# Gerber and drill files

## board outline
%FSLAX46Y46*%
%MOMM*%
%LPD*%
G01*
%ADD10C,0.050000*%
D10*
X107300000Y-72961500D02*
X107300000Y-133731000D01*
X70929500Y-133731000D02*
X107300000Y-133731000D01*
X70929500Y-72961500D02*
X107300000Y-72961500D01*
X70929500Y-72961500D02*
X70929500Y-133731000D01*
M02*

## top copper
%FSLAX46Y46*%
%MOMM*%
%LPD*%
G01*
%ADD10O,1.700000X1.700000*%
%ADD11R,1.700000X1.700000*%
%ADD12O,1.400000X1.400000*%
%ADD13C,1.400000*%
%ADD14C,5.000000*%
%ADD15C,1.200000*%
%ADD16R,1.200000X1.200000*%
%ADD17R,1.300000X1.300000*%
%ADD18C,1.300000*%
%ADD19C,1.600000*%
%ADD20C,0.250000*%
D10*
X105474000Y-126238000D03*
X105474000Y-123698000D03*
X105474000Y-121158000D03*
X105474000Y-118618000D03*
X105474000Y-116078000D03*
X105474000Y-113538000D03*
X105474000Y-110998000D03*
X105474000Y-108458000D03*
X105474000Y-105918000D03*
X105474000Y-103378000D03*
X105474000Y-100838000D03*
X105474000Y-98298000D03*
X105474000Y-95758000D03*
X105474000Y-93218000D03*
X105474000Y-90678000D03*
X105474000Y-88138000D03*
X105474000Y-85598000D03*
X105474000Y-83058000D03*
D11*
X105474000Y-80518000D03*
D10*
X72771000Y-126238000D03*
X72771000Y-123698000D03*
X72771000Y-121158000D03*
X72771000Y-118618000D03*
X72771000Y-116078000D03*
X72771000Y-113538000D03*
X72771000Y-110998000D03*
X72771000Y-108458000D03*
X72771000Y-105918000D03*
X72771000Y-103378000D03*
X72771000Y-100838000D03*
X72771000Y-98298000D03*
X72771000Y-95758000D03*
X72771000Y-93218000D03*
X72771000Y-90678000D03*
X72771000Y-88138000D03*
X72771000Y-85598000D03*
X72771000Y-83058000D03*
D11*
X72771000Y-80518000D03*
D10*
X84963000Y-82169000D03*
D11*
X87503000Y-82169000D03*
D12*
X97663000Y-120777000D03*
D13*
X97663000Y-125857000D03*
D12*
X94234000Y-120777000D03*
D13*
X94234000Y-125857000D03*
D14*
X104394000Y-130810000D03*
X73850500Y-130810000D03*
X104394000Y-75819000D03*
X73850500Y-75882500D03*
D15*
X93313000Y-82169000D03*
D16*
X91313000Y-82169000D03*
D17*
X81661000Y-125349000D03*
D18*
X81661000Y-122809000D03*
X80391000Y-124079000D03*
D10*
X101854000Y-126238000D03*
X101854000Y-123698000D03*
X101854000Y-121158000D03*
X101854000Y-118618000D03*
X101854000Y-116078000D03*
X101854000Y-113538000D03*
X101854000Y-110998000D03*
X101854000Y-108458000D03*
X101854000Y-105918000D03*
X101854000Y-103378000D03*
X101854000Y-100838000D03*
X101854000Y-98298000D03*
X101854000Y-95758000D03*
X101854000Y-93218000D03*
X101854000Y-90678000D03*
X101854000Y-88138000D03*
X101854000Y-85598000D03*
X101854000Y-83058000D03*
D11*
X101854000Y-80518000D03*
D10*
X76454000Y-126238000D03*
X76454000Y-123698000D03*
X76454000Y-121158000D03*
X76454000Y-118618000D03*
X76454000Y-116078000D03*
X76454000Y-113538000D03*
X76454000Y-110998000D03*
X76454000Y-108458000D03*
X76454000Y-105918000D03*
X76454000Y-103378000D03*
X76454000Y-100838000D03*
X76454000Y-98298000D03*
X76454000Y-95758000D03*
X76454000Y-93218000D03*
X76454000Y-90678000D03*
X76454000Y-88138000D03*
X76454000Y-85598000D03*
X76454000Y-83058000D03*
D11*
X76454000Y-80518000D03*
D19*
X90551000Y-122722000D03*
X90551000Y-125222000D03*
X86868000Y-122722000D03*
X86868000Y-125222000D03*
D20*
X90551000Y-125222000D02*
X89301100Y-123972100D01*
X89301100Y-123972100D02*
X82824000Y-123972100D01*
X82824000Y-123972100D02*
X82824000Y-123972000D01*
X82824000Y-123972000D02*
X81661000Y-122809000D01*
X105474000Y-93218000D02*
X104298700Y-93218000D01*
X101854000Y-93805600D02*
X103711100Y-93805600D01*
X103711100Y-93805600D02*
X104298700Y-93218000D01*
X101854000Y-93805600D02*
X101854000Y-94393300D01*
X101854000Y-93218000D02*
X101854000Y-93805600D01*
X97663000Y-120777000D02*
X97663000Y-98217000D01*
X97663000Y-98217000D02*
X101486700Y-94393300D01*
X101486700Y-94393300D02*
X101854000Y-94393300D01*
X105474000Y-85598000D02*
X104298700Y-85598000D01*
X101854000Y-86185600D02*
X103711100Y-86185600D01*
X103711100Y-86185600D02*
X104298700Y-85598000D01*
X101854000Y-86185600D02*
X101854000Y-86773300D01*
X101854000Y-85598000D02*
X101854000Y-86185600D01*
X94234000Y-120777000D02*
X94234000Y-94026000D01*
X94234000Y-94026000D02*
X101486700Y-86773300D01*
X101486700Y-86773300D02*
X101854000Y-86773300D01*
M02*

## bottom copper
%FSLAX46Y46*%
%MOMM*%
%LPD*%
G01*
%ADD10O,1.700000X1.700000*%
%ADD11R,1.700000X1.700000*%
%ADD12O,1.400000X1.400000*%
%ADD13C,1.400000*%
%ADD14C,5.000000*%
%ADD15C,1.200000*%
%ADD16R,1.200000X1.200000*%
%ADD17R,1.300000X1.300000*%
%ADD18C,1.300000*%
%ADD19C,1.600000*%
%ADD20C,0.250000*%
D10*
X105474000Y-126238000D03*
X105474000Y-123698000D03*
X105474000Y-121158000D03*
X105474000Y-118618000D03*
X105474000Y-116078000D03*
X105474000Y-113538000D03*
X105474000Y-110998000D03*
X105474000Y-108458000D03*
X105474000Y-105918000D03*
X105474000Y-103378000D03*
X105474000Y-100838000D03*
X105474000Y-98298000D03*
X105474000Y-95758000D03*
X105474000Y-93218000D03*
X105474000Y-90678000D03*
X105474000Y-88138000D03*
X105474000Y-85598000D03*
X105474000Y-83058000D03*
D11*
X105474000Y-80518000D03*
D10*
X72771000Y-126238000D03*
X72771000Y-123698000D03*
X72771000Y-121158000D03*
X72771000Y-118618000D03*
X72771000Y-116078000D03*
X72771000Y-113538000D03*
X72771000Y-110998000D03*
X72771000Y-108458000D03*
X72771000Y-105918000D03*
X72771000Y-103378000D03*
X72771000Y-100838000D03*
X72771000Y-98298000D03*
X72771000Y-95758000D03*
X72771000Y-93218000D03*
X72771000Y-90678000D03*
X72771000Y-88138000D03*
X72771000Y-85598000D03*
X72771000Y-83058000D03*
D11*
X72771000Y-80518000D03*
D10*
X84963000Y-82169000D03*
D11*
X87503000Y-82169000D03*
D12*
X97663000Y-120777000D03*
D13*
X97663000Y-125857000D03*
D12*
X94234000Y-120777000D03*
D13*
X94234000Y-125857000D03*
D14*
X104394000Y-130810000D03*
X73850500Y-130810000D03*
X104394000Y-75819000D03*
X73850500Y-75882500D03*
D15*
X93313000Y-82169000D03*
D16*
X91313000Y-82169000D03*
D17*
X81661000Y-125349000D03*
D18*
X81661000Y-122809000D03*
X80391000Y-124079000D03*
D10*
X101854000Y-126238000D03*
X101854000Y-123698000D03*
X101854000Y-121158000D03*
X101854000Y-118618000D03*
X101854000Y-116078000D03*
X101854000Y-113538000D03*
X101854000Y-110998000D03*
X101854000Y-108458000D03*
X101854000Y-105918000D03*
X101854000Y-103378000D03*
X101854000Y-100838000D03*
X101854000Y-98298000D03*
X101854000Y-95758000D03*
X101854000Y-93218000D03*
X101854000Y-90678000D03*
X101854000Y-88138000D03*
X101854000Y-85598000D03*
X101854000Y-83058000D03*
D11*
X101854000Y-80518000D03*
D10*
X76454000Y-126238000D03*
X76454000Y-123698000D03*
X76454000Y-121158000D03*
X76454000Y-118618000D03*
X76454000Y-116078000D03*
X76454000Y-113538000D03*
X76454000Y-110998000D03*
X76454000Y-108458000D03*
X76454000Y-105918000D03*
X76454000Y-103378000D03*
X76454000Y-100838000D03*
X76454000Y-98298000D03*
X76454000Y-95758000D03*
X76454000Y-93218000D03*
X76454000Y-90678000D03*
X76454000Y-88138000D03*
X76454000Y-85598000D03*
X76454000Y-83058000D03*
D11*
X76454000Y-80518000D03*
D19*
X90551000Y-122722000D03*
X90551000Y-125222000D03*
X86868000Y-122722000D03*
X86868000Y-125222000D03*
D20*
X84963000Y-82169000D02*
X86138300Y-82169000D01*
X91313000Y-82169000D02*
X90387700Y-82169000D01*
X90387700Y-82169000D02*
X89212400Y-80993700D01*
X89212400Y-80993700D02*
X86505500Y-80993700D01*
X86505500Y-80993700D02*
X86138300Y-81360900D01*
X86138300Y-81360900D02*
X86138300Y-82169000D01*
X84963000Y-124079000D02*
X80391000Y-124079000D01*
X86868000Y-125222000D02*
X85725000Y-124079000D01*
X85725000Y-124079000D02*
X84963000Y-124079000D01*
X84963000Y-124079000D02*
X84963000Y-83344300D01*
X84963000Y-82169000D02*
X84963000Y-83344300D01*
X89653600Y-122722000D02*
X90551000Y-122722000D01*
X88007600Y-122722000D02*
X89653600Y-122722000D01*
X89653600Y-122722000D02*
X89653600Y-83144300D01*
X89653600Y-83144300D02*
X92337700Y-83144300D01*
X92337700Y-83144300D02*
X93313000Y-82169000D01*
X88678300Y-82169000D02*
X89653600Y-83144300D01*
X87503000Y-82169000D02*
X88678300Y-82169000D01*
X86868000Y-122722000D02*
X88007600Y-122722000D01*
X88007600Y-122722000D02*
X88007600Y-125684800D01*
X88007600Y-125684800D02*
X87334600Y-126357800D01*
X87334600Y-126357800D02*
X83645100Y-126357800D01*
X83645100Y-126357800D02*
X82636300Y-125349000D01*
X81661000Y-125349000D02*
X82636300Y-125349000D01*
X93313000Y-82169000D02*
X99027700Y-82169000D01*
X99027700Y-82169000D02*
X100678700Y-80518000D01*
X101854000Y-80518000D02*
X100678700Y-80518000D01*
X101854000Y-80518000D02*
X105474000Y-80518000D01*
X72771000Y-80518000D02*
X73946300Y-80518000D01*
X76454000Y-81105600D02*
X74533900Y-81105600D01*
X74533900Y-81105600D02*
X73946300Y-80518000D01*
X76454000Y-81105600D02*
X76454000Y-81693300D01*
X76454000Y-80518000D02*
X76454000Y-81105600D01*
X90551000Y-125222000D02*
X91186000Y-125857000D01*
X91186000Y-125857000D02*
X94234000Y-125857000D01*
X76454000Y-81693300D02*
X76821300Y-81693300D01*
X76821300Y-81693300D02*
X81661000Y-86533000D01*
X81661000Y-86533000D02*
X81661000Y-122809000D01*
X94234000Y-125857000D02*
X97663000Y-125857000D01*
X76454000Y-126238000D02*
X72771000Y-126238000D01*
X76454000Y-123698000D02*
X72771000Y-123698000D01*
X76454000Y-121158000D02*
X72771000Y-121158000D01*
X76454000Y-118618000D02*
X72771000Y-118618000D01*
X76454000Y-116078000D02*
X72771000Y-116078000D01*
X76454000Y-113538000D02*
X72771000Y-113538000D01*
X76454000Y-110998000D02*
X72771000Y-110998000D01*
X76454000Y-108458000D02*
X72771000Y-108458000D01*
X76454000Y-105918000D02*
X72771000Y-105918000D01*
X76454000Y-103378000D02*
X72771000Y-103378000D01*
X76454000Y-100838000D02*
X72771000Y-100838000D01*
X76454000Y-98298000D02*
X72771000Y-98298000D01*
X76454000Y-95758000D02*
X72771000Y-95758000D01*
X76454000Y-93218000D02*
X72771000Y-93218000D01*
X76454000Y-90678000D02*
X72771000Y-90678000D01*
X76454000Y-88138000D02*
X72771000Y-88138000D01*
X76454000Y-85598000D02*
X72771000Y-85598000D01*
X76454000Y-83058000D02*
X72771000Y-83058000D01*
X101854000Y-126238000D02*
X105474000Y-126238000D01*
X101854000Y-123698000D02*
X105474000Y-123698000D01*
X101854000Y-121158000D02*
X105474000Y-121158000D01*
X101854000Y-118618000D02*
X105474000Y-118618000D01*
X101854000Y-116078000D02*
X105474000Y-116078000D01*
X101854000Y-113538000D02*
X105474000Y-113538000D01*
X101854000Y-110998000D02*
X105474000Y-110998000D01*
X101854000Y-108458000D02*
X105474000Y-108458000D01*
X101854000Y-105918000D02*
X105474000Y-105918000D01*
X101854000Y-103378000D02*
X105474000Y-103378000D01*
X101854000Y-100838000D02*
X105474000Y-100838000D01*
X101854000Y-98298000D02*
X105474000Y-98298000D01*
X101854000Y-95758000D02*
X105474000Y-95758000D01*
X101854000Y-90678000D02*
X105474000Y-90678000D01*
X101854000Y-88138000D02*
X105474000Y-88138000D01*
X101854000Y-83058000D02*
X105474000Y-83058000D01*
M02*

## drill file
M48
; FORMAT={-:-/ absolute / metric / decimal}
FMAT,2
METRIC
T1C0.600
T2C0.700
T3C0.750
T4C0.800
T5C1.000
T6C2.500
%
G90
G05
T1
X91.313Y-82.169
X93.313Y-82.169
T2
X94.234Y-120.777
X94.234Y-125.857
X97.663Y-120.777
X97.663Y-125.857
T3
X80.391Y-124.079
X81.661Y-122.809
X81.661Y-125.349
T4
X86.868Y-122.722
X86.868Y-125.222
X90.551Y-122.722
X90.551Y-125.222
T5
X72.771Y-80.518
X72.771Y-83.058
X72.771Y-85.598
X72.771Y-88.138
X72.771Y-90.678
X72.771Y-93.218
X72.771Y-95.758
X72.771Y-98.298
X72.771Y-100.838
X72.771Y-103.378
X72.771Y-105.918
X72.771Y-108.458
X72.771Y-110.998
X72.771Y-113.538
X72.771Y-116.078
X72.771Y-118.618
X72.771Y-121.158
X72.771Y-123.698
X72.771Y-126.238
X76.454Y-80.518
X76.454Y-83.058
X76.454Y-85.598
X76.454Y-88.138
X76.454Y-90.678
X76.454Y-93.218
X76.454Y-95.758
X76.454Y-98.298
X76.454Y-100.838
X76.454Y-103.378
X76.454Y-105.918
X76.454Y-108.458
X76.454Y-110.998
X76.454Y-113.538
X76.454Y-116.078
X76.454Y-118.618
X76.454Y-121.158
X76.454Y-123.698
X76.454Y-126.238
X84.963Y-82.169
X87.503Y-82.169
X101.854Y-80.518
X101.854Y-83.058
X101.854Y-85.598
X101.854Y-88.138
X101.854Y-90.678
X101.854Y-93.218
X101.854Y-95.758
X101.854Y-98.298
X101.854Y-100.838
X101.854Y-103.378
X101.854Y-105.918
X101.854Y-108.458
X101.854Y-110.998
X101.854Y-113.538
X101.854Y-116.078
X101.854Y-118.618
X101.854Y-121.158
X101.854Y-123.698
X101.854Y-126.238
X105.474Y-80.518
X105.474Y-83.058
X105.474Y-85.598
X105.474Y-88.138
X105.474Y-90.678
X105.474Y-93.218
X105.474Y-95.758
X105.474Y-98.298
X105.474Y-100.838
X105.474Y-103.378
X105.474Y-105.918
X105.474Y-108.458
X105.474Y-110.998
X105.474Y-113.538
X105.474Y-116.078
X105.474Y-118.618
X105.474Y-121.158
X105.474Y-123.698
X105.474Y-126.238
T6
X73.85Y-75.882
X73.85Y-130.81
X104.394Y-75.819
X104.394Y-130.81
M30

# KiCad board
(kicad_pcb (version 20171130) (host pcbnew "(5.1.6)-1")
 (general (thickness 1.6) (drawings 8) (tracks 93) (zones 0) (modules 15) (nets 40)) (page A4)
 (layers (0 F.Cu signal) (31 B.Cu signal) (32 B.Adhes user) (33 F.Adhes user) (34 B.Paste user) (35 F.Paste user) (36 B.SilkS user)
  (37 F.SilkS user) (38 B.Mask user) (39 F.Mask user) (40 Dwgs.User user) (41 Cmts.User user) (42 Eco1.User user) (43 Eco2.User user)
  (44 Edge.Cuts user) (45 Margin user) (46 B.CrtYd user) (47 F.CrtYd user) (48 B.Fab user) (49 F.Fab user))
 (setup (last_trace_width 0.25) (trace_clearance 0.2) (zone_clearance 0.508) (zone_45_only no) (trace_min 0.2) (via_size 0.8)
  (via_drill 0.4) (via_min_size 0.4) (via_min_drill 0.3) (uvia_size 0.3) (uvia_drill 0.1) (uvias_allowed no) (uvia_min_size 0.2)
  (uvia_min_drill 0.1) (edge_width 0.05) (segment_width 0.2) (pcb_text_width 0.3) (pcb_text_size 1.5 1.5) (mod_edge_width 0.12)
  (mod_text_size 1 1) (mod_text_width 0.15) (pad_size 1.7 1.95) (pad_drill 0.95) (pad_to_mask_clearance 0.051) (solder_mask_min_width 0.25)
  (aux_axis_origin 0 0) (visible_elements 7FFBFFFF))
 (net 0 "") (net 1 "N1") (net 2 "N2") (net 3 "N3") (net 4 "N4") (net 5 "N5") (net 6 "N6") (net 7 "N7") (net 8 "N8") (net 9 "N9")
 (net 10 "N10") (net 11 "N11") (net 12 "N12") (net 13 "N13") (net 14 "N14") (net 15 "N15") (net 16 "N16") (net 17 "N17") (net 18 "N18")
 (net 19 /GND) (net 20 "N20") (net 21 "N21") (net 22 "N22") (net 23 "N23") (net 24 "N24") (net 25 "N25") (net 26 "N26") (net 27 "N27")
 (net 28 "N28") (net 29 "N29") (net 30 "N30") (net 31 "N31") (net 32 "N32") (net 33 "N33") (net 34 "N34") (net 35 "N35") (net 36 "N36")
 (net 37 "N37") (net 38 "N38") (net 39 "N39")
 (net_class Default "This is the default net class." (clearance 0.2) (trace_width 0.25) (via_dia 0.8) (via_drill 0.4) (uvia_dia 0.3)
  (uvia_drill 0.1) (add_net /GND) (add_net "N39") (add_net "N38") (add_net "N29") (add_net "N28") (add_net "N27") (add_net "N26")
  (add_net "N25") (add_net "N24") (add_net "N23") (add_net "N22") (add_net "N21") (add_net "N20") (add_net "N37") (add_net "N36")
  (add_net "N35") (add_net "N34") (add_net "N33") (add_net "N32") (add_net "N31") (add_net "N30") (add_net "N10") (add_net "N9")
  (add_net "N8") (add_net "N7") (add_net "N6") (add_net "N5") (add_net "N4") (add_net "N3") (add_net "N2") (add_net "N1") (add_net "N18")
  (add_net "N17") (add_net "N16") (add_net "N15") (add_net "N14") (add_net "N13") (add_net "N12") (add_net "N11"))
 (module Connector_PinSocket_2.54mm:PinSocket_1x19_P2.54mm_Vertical (layer F.Cu) (at 105.474 80.518)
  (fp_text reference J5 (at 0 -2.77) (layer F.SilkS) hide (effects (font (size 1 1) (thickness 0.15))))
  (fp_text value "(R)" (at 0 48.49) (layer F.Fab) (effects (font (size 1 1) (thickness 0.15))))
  (pad 19 thru_hole oval (at 0 45.72) (size 1.7 1.7) (drill 1) (layers *.Cu *.Mask) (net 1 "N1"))
  (pad 18 thru_hole oval (at 0 43.18) (size 1.7 1.7) (drill 1) (layers *.Cu *.Mask) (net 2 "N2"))
  (pad 17 thru_hole oval (at 0 40.64) (size 1.7 1.7) (drill 1) (layers *.Cu *.Mask) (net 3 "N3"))
  (pad 16 thru_hole oval (at 0 38.1) (size 1.7 1.7) (drill 1) (layers *.Cu *.Mask) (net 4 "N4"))
  (pad 15 thru_hole oval (at 0 35.56) (size 1.7 1.7) (drill 1) (layers *.Cu *.Mask) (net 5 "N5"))
  (pad 14 thru_hole oval (at 0 33.02) (size 1.7 1.7) (drill 1) (layers *.Cu *.Mask) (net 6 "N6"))
  (pad 13 thru_hole oval (at 0 30.48) (size 1.7 1.7) (drill 1) (layers *.Cu *.Mask) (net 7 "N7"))
  (pad 12 thru_hole oval (at 0 27.94) (size 1.7 1.7) (drill 1) (layers *.Cu *.Mask) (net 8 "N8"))
  (pad 11 thru_hole oval (at 0 25.4) (size 1.7 1.7) (drill 1) (layers *.Cu *.Mask) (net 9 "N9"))
  (pad 10 thru_hole oval (at 0 22.86) (size 1.7 1.7) (drill 1) (layers *.Cu *.Mask) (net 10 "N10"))
  (pad 9 thru_hole oval (at 0 20.32) (size 1.7 1.7) (drill 1) (layers *.Cu *.Mask) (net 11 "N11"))
  (pad 8 thru_hole oval (at 0 17.78) (size 1.7 1.7) (drill 1) (layers *.Cu *.Mask) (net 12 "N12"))
  (pad 7 thru_hole oval (at 0 15.24) (size 1.7 1.7) (drill 1) (layers *.Cu *.Mask) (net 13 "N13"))
  (pad 6 thru_hole oval (at 0 12.7) (size 1.7 1.7) (drill 1) (layers *.Cu *.Mask) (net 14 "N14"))
  (pad 5 thru_hole oval (at 0 10.16) (size 1.7 1.7) (drill 1) (layers *.Cu *.Mask) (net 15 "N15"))
  (pad 4 thru_hole oval (at 0 7.62) (size 1.7 1.7) (drill 1) (layers *.Cu *.Mask) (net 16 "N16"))
  (pad 3 thru_hole oval (at 0 5.08) (size 1.7 1.7) (drill 1) (layers *.Cu *.Mask) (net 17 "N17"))
  (pad 2 thru_hole oval (at 0 2.54) (size 1.7 1.7) (drill 1) (layers *.Cu *.Mask) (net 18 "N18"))
  (pad 1 thru_hole rect (at 0 0) (size 1.7 1.7) (drill 1) (layers *.Cu *.Mask) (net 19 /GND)))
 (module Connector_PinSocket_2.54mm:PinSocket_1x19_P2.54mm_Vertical (layer F.Cu) (at 72.771 80.518)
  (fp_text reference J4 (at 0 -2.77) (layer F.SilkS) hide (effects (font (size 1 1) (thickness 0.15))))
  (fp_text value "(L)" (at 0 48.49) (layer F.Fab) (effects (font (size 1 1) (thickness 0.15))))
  (pad 19 thru_hole oval (at 0 45.72) (size 1.7 1.7) (drill 1) (layers *.Cu *.Mask) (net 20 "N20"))
  (pad 18 thru_hole oval (at 0 43.18) (size 1.7 1.7) (drill 1) (layers *.Cu *.Mask) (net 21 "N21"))
  (pad 17 thru_hole oval (at 0 40.64) (size 1.7 1.7) (drill 1) (layers *.Cu *.Mask) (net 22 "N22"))
  (pad 16 thru_hole oval (at 0 38.1) (size 1.7 1.7) (drill 1) (layers *.Cu *.Mask) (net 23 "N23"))
  (pad 15 thru_hole oval (at 0 35.56) (size 1.7 1.7) (drill 1) (layers *.Cu *.Mask) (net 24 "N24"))
  (pad 14 thru_hole oval (at 0 33.02) (size 1.7 1.7) (drill 1) (layers *.Cu *.Mask) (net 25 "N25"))
  (pad 13 thru_hole oval (at 0 30.48) (size 1.7 1.7) (drill 1) (layers *.Cu *.Mask) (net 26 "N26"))
  (pad 12 thru_hole oval (at 0 27.94) (size 1.7 1.7) (drill 1) (layers *.Cu *.Mask) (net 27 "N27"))
  (pad 11 thru_hole oval (at 0 25.4) (size 1.7 1.7) (drill 1) (layers *.Cu *.Mask) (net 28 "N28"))
  (pad 10 thru_hole oval (at 0 22.86) (size 1.7 1.7) (drill 1) (layers *.Cu *.Mask) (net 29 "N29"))
  (pad 9 thru_hole oval (at 0 20.32) (size 1.7 1.7) (drill 1) (layers *.Cu *.Mask) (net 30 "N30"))
  (pad 8 thru_hole oval (at 0 17.78) (size 1.7 1.7) (drill 1) (layers *.Cu *.Mask) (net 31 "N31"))
  (pad 7 thru_hole oval (at 0 15.24) (size 1.7 1.7) (drill 1) (layers *.Cu *.Mask) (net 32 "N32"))
  (pad 6 thru_hole oval (at 0 12.7) (size 1.7 1.7) (drill 1) (layers *.Cu *.Mask) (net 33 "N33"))
  (pad 5 thru_hole oval (at 0 10.16) (size 1.7 1.7) (drill 1) (layers *.Cu *.Mask) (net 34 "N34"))
  (pad 4 thru_hole oval (at 0 7.62) (size 1.7 1.7) (drill 1) (layers *.Cu *.Mask) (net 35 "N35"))
  (pad 3 thru_hole oval (at 0 5.08) (size 1.7 1.7) (drill 1) (layers *.Cu *.Mask) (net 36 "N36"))
  (pad 2 thru_hole oval (at 0 2.54) (size 1.7 1.7) (drill 1) (layers *.Cu *.Mask) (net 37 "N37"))
  (pad 1 thru_hole rect (at 0 0) (size 1.7 1.7) (drill 1) (layers *.Cu *.Mask) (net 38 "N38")))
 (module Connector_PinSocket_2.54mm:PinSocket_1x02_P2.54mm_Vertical (layer F.Cu) (at 87.503 82.169 270)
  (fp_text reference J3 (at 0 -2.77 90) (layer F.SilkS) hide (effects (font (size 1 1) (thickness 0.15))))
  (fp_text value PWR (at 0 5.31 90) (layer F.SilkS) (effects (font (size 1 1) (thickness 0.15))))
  (pad 2 thru_hole oval (at 0 2.54 270) (size 1.7 1.7) (drill 1) (layers *.Cu *.Mask) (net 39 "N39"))
  (pad 1 thru_hole rect (at 0 0 270) (size 1.7 1.7) (drill 1) (layers *.Cu *.Mask) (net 19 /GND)))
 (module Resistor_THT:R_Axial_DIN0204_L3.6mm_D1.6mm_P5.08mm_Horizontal (layer F.Cu) (at 97.663 125.857 90)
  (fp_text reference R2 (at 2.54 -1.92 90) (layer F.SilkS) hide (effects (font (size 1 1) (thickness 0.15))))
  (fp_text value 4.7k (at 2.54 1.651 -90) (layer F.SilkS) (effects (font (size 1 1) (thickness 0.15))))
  (pad 2 thru_hole oval (at 5.08 0 90) (size 1.4 1.4) (drill 0.7) (layers *.Cu *.Mask) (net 14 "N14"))
  (pad 1 thru_hole circle (at 0 0 90) (size 1.4 1.4) (drill 0.7) (layers *.Cu *.Mask) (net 38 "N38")))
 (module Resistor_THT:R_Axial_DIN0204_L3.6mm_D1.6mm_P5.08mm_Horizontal (layer F.Cu) (at 94.234 125.857 90)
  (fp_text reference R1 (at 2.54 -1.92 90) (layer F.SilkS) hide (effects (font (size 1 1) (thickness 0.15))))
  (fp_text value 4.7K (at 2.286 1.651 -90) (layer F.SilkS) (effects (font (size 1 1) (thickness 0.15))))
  (pad 2 thru_hole oval (at 5.08 0 90) (size 1.4 1.4) (drill 0.7) (layers *.Cu *.Mask) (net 17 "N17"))
  (pad 1 thru_hole circle (at 0 0 90) (size 1.4 1.4) (drill 0.7) (layers *.Cu *.Mask) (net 38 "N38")))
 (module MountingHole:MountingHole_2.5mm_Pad (layer F.Cu) (at 104.394 130.81)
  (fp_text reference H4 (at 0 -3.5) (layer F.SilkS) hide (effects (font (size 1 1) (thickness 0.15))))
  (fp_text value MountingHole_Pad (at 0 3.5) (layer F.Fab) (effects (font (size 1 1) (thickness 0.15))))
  (pad 1 thru_hole circle (at 0 0) (size 5 5) (drill 2.5) (layers *.Cu *.Mask)))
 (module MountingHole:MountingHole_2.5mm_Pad (layer F.Cu) (at 73.8505 130.81)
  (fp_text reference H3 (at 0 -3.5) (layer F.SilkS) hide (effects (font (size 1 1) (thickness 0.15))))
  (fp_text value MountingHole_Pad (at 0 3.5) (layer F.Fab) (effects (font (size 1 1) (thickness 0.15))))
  (pad 1 thru_hole circle (at 0 0) (size 5 5) (drill 2.5) (layers *.Cu *.Mask)))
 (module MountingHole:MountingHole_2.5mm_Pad (layer F.Cu) (at 104.394 75.819)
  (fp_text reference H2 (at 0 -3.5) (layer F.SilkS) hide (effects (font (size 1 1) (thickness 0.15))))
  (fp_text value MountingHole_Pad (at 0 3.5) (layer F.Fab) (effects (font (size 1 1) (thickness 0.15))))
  (pad 1 thru_hole circle (at 0 0) (size 5 5) (drill 2.5) (layers *.Cu *.Mask)))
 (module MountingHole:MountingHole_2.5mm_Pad (layer F.Cu) (at 73.8505 75.8825)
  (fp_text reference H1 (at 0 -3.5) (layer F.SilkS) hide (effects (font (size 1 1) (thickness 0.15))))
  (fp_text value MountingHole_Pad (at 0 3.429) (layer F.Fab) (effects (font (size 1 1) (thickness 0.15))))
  (pad 1 thru_hole circle (at 0 0) (size 5 5) (drill 2.5) (layers *.Cu *.Mask)))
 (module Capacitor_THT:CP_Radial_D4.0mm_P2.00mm (layer F.Cu) (at 91.313 82.169)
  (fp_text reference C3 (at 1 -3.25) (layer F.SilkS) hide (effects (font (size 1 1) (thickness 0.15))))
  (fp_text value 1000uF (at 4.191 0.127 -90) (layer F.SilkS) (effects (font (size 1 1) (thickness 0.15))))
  (pad 2 thru_hole circle (at 2 0) (size 1.2 1.2) (drill 0.6) (layers *.Cu *.Mask) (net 19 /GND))
  (pad 1 thru_hole rect (at 0 0) (size 1.2 1.2) (drill 0.6) (layers *.Cu *.Mask) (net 39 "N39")))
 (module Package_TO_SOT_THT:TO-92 (layer F.Cu) (at 81.661 125.349 90)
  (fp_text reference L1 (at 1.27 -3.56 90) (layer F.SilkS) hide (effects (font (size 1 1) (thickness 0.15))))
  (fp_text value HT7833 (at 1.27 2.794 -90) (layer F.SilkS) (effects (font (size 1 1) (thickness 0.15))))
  (pad 1 thru_hole rect (at 0 0 180) (size 1.3 1.3) (drill 0.75) (layers *.Cu *.Mask) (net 19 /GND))
  (pad 3 thru_hole circle (at 2.54 0 180) (size 1.3 1.3) (drill 0.75) (layers *.Cu *.Mask) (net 38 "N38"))
  (pad 2 thru_hole circle (at 1.27 -1.27 180) (size 1.3 1.3) (drill 0.75) (layers *.Cu *.Mask) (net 39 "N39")))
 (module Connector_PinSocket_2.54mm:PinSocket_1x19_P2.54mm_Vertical (layer F.Cu) (at 101.854 80.518)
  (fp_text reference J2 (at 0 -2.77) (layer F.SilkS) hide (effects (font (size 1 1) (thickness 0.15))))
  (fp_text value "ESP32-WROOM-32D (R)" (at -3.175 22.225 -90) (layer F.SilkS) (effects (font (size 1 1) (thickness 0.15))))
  (pad 19 thru_hole oval (at 0 45.72) (size 1.7 1.7) (drill 1) (layers *.Cu *.Mask) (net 1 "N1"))
  (pad 18 thru_hole oval (at 0 43.18) (size 1.7 1.7) (drill 1) (layers *.Cu *.Mask) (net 2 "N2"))
  (pad 17 thru_hole oval (at 0 40.64) (size 1.7 1.7) (drill 1) (layers *.Cu *.Mask) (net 3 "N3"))
  (pad 16 thru_hole oval (at 0 38.1) (size 1.7 1.7) (drill 1) (layers *.Cu *.Mask) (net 4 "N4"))
  (pad 15 thru_hole oval (at 0 35.56) (size 1.7 1.7) (drill 1) (layers *.Cu *.Mask) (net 5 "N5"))
  (pad 14 thru_hole oval (at 0 33.02) (size 1.7 1.7) (drill 1) (layers *.Cu *.Mask) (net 6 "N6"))
  (pad 13 thru_hole oval (at 0 30.48) (size 1.7 1.7) (drill 1) (layers *.Cu *.Mask) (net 7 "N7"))
  (pad 12 thru_hole oval (at 0 27.94) (size 1.7 1.7) (drill 1) (layers *.Cu *.Mask) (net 8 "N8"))
  (pad 11 thru_hole oval (at 0 25.4) (size 1.7 1.7) (drill 1) (layers *.Cu *.Mask) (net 9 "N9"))
  (pad 10 thru_hole oval (at 0 22.86) (size 1.7 1.7) (drill 1) (layers *.Cu *.Mask) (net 10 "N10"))
  (pad 9 thru_hole oval (at 0 20.32) (size 1.7 1.7) (drill 1) (layers *.Cu *.Mask) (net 11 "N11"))
  (pad 8 thru_hole oval (at 0 17.78) (size 1.7 1.7) (drill 1) (layers *.Cu *.Mask) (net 12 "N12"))
  (pad 7 thru_hole oval (at 0 15.24) (size 1.7 1.7) (drill 1) (layers *.Cu *.Mask) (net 13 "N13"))
  (pad 6 thru_hole oval (at 0 12.7) (size 1.7 1.7) (drill 1) (layers *.Cu *.Mask) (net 14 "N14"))
  (pad 5 thru_hole oval (at 0 10.16) (size 1.7 1.7) (drill 1) (layers *.Cu *.Mask) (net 15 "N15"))
  (pad 4 thru_hole oval (at 0 7.62) (size 1.7 1.7) (drill 1) (layers *.Cu *.Mask) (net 16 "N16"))
  (pad 3 thru_hole oval (at 0 5.08) (size 1.7 1.7) (drill 1) (layers *.Cu *.Mask) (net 17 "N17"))
  (pad 2 thru_hole oval (at 0 2.54) (size 1.7 1.7) (drill 1) (layers *.Cu *.Mask) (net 18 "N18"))
  (pad 1 thru_hole rect (at 0 0) (size 1.7 1.7) (drill 1) (layers *.Cu *.Mask) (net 19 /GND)))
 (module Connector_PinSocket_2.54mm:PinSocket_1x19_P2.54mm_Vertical (layer F.Cu) (at 76.454 80.518)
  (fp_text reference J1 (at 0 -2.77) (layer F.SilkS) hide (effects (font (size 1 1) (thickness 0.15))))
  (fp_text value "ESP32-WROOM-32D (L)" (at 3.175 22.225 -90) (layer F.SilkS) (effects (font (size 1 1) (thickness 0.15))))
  (pad 19 thru_hole oval (at 0 45.72) (size 1.7 1.7) (drill 1) (layers *.Cu *.Mask) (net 20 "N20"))
  (pad 18 thru_hole oval (at 0 43.18) (size 1.7 1.7) (drill 1) (layers *.Cu *.Mask) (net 21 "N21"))
  (pad 17 thru_hole oval (at 0 40.64) (size 1.7 1.7) (drill 1) (layers *.Cu *.Mask) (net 22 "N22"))
  (pad 16 thru_hole oval (at 0 38.1) (size 1.7 1.7) (drill 1) (layers *.Cu *.Mask) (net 23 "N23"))
  (pad 15 thru_hole oval (at 0 35.56) (size 1.7 1.7) (drill 1) (layers *.Cu *.Mask) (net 24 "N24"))
  (pad 14 thru_hole oval (at 0 33.02) (size 1.7 1.7) (drill 1) (layers *.Cu *.Mask) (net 25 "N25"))
  (pad 13 thru_hole oval (at 0 30.48) (size 1.7 1.7) (drill 1) (layers *.Cu *.Mask) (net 26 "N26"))
  (pad 12 thru_hole oval (at 0 27.94) (size 1.7 1.7) (drill 1) (layers *.Cu *.Mask) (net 27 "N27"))
  (pad 11 thru_hole oval (at 0 25.4) (size 1.7 1.7) (drill 1) (layers *.Cu *.Mask) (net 28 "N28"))
  (pad 10 thru_hole oval (at 0 22.86) (size 1.7 1.7) (drill 1) (layers *.Cu *.Mask) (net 29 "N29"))
  (pad 9 thru_hole oval (at 0 20.32) (size 1.7 1.7) (drill 1) (layers *.Cu *.Mask) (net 30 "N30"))
  (pad 8 thru_hole oval (at 0 17.78) (size 1.7 1.7) (drill 1) (layers *.Cu *.Mask) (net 31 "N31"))
  (pad 7 thru_hole oval (at 0 15.24) (size 1.7 1.7) (drill 1) (layers *.Cu *.Mask) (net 32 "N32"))
  (pad 6 thru_hole oval (at 0 12.7) (size 1.7 1.7) (drill 1) (layers *.Cu *.Mask) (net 33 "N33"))
  (pad 5 thru_hole oval (at 0 10.16) (size 1.7 1.7) (drill 1) (layers *.Cu *.Mask) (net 34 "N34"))
  (pad 4 thru_hole oval (at 0 7.62) (size 1.7 1.7) (drill 1) (layers *.Cu *.Mask) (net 35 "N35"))
  (pad 3 thru_hole oval (at 0 5.08) (size 1.7 1.7) (drill 1) (layers *.Cu *.Mask) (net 36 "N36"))
  (pad 2 thru_hole oval (at 0 2.54) (size 1.7 1.7) (drill 1) (layers *.Cu *.Mask) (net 37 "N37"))
  (pad 1 thru_hole rect (at 0 0) (size 1.7 1.7) (drill 1) (layers *.Cu *.Mask) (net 38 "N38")))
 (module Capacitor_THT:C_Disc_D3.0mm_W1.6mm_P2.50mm (layer F.Cu) (at 90.551 125.222 90)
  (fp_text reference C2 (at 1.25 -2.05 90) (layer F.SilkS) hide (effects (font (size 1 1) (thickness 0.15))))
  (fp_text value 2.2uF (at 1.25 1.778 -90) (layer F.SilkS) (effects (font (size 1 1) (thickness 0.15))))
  (pad 2 thru_hole circle (at 2.5 0 90) (size 1.6 1.6) (drill 0.8) (layers *.Cu *.Mask) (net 19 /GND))
  (pad 1 thru_hole circle (at 0 0 90) (size 1.6 1.6) (drill 0.8) (layers *.Cu *.Mask) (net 38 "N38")))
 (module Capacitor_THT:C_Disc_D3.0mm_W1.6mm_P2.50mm (layer F.Cu) (at 86.868 125.222 90)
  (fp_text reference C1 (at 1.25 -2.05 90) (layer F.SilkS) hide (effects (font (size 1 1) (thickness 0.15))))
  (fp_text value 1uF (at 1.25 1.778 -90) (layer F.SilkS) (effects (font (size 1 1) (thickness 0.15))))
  (pad 2 thru_hole circle (at 2.5 0 90) (size 1.6 1.6) (drill 0.8) (layers *.Cu *.Mask) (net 19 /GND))
  (pad 1 thru_hole circle (at 0 0 90) (size 1.6 1.6) (drill 0.8) (layers *.Cu *.Mask) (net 39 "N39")))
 (gr_line (start 107.3 72.9615) (end 107.3 133.731) (layer Edge.Cuts) (width 0.05))
 (gr_line (start 70.9295 133.731) (end 107.3 133.731) (layer Edge.Cuts) (width 0.05))
 (gr_line (start 70.9295 72.9615) (end 107.3 72.9615) (layer Edge.Cuts) (width 0.05))
 (gr_line (start 70.9295 72.9615) (end 70.9295 133.731) (layer Edge.Cuts) (width 0.05))
 (segment (start 84.963 82.169) (end 86.1383 82.169) (width 0.25) (layer B.Cu) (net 39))
 (segment (start 91.313 82.169) (end 90.3877 82.169) (width 0.25) (layer B.Cu) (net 39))
 (segment (start 90.3877 82.169) (end 89.2124 80.9937) (width 0.25) (layer B.Cu) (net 39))
 (segment (start 89.2124 80.9937) (end 86.5055 80.9937) (width 0.25) (layer B.Cu) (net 39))
 (segment (start 86.5055 80.9937) (end 86.1383 81.3609) (width 0.25) (layer B.Cu) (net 39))
 (segment (start 86.1383 81.3609) (end 86.1383 82.169) (width 0.25) (layer B.Cu) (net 39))
 (segment (start 84.963 124.079) (end 80.391 124.079) (width 0.25) (layer B.Cu) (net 39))
 (segment (start 86.868 125.222) (end 85.725 124.079) (width 0.25) (layer B.Cu) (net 39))
 (segment (start 85.725 124.079) (end 84.963 124.079) (width 0.25) (layer B.Cu) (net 39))
 (segment (start 84.963 124.079) (end 84.963 83.3443) (width 0.25) (layer B.Cu) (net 39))
 (segment (start 84.963 82.169) (end 84.963 83.3443) (width 0.25) (layer B.Cu) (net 39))
 (segment (start 89.6536 122.722) (end 90.551 122.722) (width 0.25) (layer B.Cu) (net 19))
 (segment (start 88.0076 122.722) (end 89.6536 122.722) (width 0.25) (layer B.Cu) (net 19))
 (segment (start 89.6536 122.722) (end 89.6536 83.1443) (width 0.25) (layer B.Cu) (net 19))
 (segment (start 89.6536 83.1443) (end 92.3377 83.1443) (width 0.25) (layer B.Cu) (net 19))
 (segment (start 92.3377 83.1443) (end 93.313 82.169) (width 0.25) (layer B.Cu) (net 19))
 (segment (start 88.6783 82.169) (end 89.6536 83.1443) (width 0.25) (layer B.Cu) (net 19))
 (segment (start 87.503 82.169) (end 88.6783 82.169) (width 0.25) (layer B.Cu) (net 19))
 (segment (start 86.868 122.722) (end 88.0076 122.722) (width 0.25) (layer B.Cu) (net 19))
 (segment (start 88.0076 122.722) (end 88.0076 125.6848) (width 0.25) (layer B.Cu) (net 19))
 (segment (start 88.0076 125.6848) (end 87.3346 126.3578) (width 0.25) (layer B.Cu) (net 19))
 (segment (start 87.3346 126.3578) (end 83.6451 126.3578) (width 0.25) (layer B.Cu) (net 19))
 (segment (start 83.6451 126.3578) (end 82.6363 125.349) (width 0.25) (layer B.Cu) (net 19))
 (segment (start 81.661 125.349) (end 82.6363 125.349) (width 0.25) (layer B.Cu) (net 19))
 (segment (start 93.313 82.169) (end 99.0277 82.169) (width 0.25) (layer B.Cu) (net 19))
 (segment (start 99.0277 82.169) (end 100.6787 80.518) (width 0.25) (layer B.Cu) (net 19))
 (segment (start 101.854 80.518) (end 100.6787 80.518) (width 0.25) (layer B.Cu) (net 19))
 (segment (start 101.854 80.518) (end 105.474 80.518) (width 0.25) (layer B.Cu) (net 19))
 (segment (start 72.771 80.518) (end 73.9463 80.518) (width 0.25) (layer B.Cu) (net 38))
 (segment (start 76.454 81.1056) (end 74.5339 81.1056) (width 0.25) (layer B.Cu) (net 38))
 (segment (start 74.5339 81.1056) (end 73.9463 80.518) (width 0.25) (layer B.Cu) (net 38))
 (segment (start 76.454 81.1056) (end 76.454 81.6933) (width 0.25) (layer B.Cu) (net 38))
 (segment (start 76.454 80.518) (end 76.454 81.1056) (width 0.25) (layer B.Cu) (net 38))
 (segment (start 90.551 125.222) (end 91.186 125.857) (width 0.25) (layer B.Cu) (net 38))
 (segment (start 91.186 125.857) (end 94.234 125.857) (width 0.25) (layer B.Cu) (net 38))
 (segment (start 76.454 81.6933) (end 76.8213 81.6933) (width 0.25) (layer B.Cu) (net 38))
 (segment (start 76.8213 81.6933) (end 81.661 86.533) (width 0.25) (layer B.Cu) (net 38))
 (segment (start 81.661 86.533) (end 81.661 122.809) (width 0.25) (layer B.Cu) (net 38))
 (segment (start 90.551 125.222) (end 89.3011 123.9721) (width 0.25) (layer F.Cu) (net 38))
 (segment (start 89.3011 123.9721) (end 82.824 123.9721) (width 0.25) (layer F.Cu) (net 38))
 (segment (start 82.824 123.9721) (end 82.824 123.972) (width 0.25) (layer F.Cu) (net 38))
 (segment (start 82.824 123.972) (end 81.661 122.809) (width 0.25) (layer F.Cu) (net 38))
 (segment (start 94.234 125.857) (end 97.663 125.857) (width 0.25) (layer B.Cu) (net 38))
 (segment (start 76.454 126.238) (end 72.771 126.238) (width 0.25) (layer B.Cu) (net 20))
 (segment (start 76.454 123.698) (end 72.771 123.698) (width 0.25) (layer B.Cu) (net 21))
 (segment (start 76.454 121.158) (end 72.771 121.158) (width 0.25) (layer B.Cu) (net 22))
 (segment (start 76.454 118.618) (end 72.771 118.618) (width 0.25) (layer B.Cu) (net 23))
 (segment (start 76.454 116.078) (end 72.771 116.078) (width 0.25) (layer B.Cu) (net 24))
 (segment (start 76.454 113.538) (end 72.771 113.538) (width 0.25) (layer B.Cu) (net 25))
 (segment (start 76.454 110.998) (end 72.771 110.998) (width 0.25) (layer B.Cu) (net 26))
 (segment (start 76.454 108.458) (end 72.771 108.458) (width 0.25) (layer B.Cu) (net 27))
 (segment (start 76.454 105.918) (end 72.771 105.918) (width 0.25) (layer B.Cu) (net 28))
 (segment (start 76.454 103.378) (end 72.771 103.378) (width 0.25) (layer B.Cu) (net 29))
 (segment (start 76.454 100.838) (end 72.771 100.838) (width 0.25) (layer B.Cu) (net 30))
 (segment (start 76.454 98.298) (end 72.771 98.298) (width 0.25) (layer B.Cu) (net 31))
 (segment (start 76.454 95.758) (end 72.771 95.758) (width 0.25) (layer B.Cu) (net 32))
 (segment (start 76.454 93.218) (end 72.771 93.218) (width 0.25) (layer B.Cu) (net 33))
 (segment (start 76.454 90.678) (end 72.771 90.678) (width 0.25) (layer B.Cu) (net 34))
 (segment (start 76.454 88.138) (end 72.771 88.138) (width 0.25) (layer B.Cu) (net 35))
 (segment (start 76.454 85.598) (end 72.771 85.598) (width 0.25) (layer B.Cu) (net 36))
 (segment (start 76.454 83.058) (end 72.771 83.058) (width 0.25) (layer B.Cu) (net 37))
 (segment (start 101.854 126.238) (end 105.474 126.238) (width 0.25) (layer B.Cu) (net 1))
 (segment (start 101.854 123.698) (end 105.474 123.698) (width 0.25) (layer B.Cu) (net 2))
 (segment (start 101.854 121.158) (end 105.474 121.158) (width 0.25) (layer B.Cu) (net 3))
 (segment (start 101.854 118.618) (end 105.474 118.618) (width 0.25) (layer B.Cu) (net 4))
 (segment (start 101.854 116.078) (end 105.474 116.078) (width 0.25) (layer B.Cu) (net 5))
 (segment (start 101.854 113.538) (end 105.474 113.538) (width 0.25) (layer B.Cu) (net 6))
 (segment (start 101.854 110.998) (end 105.474 110.998) (width 0.25) (layer B.Cu) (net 7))
 (segment (start 101.854 108.458) (end 105.474 108.458) (width 0.25) (layer B.Cu) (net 8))
 (segment (start 101.854 105.918) (end 105.474 105.918) (width 0.25) (layer B.Cu) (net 9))
 (segment (start 101.854 103.378) (end 105.474 103.378) (width 0.25) (layer B.Cu) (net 10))
 (segment (start 101.854 100.838) (end 105.474 100.838) (width 0.25) (layer B.Cu) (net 11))
 (segment (start 101.854 98.298) (end 105.474 98.298) (width 0.25) (layer B.Cu) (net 12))
 (segment (start 101.854 95.758) (end 105.474 95.758) (width 0.25) (layer B.Cu) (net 13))
 (segment (start 105.474 93.218) (end 104.2987 93.218) (width 0.25) (layer F.Cu) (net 14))
 (segment (start 101.854 93.8056) (end 103.7111 93.8056) (width 0.25) (layer F.Cu) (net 14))
 (segment (start 103.7111 93.8056) (end 104.2987 93.218) (width 0.25) (layer F.Cu) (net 14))
 (segment (start 101.854 93.8056) (end 101.854 94.3933) (width 0.25) (layer F.Cu) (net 14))
 (segment (start 101.854 93.218) (end 101.854 93.8056) (width 0.25) (layer F.Cu) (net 14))
 (segment (start 97.663 120.777) (end 97.663 98.217) (width 0.25) (layer F.Cu) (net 14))
 (segment (start 97.663 98.217) (end 101.4867 94.3933) (width 0.25) (layer F.Cu) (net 14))
 (segment (start 101.4867 94.3933) (end 101.854 94.3933) (width 0.25) (layer F.Cu) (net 14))
 (segment (start 101.854 90.678) (end 105.474 90.678) (width 0.25) (layer B.Cu) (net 15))
 (segment (start 101.854 88.138) (end 105.474 88.138) (width 0.25) (layer B.Cu) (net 16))
 (segment (start 105.474 85.598) (end 104.2987 85.598) (width 0.25) (layer F.Cu) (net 17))
 (segment (start 101.854 86.1856) (end 103.7111 86.1856) (width 0.25) (layer F.Cu) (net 17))
 (segment (start 103.7111 86.1856) (end 104.2987 85.598) (width 0.25) (layer F.Cu) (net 17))
 (segment (start 101.854 86.1856) (end 101.854 86.7733) (width 0.25) (layer F.Cu) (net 17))
 (segment (start 101.854 85.598) (end 101.854 86.1856) (width 0.25) (layer F.Cu) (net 17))
 (segment (start 94.234 120.777) (end 94.234 94.026) (width 0.25) (layer F.Cu) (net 17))
 (segment (start 94.234 94.026) (end 101.4867 86.7733) (width 0.25) (layer F.Cu) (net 17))
 (segment (start 101.4867 86.7733) (end 101.854 86.7733) (width 0.25) (layer F.Cu) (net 17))
 (segment (start 101.854 83.058) (end 105.474 83.058) (width 0.25) (layer B.Cu) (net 18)))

